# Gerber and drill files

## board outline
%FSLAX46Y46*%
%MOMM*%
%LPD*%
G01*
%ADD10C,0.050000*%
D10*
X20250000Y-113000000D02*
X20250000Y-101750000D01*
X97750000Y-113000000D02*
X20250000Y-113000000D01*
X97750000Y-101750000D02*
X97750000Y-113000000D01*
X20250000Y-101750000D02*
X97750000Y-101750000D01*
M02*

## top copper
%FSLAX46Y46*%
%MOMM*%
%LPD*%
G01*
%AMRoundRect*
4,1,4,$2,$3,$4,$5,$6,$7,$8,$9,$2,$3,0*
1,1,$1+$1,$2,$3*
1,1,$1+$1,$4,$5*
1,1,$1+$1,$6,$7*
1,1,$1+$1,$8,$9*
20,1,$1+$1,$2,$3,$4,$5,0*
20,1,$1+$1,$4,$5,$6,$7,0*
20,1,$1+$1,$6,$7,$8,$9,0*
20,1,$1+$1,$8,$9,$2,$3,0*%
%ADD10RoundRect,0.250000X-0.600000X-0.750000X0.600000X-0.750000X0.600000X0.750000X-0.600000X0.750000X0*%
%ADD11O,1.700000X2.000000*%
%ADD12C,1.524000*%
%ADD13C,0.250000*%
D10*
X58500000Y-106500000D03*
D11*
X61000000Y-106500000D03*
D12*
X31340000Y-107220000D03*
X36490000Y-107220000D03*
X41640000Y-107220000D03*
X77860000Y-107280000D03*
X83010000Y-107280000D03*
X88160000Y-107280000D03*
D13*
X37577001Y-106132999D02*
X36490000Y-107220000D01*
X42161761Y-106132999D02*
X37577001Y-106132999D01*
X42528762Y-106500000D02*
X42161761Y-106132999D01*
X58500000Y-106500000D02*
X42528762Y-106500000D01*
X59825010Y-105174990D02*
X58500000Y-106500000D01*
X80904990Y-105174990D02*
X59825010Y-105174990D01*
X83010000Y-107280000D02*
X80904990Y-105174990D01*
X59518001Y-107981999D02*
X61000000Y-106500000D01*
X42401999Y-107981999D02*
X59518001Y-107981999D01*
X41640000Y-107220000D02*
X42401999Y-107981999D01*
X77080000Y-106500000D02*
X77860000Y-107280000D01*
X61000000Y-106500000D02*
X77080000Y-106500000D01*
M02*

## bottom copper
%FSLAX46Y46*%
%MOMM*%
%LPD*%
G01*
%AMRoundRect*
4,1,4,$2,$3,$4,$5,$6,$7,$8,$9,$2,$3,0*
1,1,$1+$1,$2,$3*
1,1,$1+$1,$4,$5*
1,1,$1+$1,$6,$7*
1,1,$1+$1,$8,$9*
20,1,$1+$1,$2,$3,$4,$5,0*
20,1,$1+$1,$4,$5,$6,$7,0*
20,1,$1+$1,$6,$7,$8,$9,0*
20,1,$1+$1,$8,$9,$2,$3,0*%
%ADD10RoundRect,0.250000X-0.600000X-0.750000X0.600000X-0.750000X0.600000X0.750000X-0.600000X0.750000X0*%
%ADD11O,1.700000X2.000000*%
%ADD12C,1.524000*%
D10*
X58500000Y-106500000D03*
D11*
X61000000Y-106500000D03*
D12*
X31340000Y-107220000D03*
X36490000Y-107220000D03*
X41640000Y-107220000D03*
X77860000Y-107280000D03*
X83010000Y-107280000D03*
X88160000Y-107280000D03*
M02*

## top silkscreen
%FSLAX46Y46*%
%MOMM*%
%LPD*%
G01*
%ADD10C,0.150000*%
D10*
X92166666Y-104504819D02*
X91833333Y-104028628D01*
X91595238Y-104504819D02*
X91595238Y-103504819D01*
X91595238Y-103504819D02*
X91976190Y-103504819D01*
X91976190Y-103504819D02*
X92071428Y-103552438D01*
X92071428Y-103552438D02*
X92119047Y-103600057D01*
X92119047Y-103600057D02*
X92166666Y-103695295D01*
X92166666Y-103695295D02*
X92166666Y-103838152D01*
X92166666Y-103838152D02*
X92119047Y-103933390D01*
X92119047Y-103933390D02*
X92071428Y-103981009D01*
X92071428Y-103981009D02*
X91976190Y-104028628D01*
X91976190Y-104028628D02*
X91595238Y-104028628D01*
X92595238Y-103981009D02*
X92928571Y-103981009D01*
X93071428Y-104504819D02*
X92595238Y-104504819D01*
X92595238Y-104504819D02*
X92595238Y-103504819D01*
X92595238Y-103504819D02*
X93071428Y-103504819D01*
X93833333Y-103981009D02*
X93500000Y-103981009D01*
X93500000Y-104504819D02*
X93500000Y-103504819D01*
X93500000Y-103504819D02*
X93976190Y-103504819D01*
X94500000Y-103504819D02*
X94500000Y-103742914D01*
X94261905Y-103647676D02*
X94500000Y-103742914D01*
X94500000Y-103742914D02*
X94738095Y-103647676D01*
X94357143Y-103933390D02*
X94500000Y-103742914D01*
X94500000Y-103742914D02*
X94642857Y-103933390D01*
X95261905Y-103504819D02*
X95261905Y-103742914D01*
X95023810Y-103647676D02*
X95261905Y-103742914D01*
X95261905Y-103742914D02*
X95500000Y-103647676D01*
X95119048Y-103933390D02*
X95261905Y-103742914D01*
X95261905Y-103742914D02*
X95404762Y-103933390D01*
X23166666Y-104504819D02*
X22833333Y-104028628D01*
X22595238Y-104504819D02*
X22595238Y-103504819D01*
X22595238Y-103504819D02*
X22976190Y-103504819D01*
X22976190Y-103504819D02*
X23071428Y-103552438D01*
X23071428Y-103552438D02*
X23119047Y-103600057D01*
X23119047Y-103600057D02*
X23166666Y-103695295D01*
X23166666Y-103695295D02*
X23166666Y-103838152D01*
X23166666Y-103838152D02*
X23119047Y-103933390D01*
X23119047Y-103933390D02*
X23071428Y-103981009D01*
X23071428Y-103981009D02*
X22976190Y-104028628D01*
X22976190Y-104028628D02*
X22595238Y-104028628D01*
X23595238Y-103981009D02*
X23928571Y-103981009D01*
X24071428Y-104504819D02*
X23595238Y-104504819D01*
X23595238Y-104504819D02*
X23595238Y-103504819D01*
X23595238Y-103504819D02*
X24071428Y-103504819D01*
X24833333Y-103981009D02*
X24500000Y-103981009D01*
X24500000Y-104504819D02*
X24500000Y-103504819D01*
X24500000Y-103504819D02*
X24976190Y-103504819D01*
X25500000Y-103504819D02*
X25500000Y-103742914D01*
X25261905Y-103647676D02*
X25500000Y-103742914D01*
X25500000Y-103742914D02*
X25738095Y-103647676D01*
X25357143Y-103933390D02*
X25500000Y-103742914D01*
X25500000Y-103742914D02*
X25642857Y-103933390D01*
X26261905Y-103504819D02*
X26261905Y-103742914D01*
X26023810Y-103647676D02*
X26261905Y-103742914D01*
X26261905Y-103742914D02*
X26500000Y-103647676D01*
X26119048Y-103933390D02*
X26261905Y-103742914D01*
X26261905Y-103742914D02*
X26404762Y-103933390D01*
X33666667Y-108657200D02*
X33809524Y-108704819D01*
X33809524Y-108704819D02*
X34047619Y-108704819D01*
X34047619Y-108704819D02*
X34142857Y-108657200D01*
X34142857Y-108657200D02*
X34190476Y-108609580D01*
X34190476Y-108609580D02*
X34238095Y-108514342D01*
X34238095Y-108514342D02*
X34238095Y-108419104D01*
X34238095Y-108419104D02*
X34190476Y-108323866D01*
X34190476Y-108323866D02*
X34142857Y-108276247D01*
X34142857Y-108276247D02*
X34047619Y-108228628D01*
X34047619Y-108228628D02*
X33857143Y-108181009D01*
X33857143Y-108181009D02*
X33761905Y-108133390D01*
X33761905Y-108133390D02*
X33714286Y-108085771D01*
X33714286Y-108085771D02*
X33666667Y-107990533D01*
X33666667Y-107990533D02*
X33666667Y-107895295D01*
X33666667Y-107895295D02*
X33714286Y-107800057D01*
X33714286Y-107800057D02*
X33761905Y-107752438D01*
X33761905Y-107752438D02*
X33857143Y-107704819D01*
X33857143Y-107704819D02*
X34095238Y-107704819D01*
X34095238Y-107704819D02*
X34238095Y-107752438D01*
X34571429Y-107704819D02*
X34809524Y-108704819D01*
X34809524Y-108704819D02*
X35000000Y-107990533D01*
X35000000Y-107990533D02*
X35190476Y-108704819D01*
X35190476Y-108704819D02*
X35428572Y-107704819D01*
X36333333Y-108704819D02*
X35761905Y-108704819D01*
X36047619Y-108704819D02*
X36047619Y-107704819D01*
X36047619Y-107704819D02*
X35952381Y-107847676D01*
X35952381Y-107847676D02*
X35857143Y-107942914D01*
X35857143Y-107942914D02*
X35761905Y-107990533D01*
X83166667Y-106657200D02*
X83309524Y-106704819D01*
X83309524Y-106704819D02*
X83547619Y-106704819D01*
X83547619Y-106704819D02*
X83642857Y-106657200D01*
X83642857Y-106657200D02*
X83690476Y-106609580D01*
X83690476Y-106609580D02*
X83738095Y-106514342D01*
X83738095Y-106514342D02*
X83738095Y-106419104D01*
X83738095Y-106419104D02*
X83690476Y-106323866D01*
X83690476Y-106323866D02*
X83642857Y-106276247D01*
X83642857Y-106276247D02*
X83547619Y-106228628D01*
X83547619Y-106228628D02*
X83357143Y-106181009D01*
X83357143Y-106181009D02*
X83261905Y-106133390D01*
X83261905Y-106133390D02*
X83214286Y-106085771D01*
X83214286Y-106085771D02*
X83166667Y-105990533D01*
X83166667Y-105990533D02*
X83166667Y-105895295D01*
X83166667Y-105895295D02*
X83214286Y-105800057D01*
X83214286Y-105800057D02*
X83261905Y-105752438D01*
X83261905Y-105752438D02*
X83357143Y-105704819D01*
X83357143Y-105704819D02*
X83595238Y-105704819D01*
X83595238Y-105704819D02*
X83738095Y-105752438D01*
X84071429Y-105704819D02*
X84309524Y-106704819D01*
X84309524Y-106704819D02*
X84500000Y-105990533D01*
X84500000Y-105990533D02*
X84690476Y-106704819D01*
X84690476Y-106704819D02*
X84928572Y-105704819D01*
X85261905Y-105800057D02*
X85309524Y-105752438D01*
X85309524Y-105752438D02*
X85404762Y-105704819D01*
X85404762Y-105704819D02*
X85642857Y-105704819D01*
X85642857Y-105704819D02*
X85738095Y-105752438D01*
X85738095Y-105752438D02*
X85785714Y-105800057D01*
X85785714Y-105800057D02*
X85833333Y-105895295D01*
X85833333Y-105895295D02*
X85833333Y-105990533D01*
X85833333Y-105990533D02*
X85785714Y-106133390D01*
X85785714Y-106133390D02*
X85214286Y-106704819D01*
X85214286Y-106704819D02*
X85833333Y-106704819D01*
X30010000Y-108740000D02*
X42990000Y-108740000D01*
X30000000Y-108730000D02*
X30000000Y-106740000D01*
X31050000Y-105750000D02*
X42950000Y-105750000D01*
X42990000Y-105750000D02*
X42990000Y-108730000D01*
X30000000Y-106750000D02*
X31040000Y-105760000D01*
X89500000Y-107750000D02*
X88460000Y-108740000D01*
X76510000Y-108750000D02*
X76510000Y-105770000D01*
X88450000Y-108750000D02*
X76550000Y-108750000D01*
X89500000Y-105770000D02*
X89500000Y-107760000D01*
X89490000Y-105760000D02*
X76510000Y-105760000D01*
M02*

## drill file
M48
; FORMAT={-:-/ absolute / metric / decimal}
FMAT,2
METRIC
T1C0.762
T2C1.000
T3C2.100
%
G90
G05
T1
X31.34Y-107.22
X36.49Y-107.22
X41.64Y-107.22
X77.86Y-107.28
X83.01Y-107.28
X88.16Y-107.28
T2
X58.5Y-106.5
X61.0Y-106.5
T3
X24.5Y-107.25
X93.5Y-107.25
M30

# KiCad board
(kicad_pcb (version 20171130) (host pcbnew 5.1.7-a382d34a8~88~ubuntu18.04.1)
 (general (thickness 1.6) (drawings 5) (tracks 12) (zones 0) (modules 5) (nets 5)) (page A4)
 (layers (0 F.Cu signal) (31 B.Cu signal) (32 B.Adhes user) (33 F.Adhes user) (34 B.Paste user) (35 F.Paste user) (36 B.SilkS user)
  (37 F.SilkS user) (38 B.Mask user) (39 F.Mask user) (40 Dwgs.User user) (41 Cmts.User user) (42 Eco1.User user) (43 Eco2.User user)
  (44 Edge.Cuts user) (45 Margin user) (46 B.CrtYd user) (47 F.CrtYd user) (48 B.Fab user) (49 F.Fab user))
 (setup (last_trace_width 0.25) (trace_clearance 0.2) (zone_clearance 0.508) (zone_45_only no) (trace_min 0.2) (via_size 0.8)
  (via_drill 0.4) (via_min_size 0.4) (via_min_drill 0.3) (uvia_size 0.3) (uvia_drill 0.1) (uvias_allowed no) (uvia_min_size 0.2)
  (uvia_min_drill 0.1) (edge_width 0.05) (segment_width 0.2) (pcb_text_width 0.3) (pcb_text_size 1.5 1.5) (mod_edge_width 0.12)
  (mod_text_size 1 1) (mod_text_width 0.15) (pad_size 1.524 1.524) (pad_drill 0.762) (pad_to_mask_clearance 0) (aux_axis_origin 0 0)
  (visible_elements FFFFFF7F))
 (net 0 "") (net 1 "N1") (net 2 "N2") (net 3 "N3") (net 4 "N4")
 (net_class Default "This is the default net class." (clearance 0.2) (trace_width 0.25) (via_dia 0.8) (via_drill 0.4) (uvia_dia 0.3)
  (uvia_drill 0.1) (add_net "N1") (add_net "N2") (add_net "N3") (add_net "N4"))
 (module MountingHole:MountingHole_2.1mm (layer F.Cu) (at 93.5 107.25)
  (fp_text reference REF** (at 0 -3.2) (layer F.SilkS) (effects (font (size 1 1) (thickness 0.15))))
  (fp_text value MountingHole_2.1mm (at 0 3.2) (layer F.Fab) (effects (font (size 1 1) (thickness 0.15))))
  (pad "" np_thru_hole circle (at 0 0) (size 2.1 2.1) (drill 2.1) (layers *.Cu *.Mask)))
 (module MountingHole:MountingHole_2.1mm (layer F.Cu) (at 24.5 107.25)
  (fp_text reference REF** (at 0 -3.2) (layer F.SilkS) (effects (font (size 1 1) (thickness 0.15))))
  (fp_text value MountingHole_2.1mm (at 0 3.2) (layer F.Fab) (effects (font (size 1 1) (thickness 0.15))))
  (pad "" np_thru_hole circle (at 0 0) (size 2.1 2.1) (drill 2.1) (layers *.Cu *.Mask)))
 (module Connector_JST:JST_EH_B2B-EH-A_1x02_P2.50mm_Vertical (layer B.Cu) (at 58.5 106.5)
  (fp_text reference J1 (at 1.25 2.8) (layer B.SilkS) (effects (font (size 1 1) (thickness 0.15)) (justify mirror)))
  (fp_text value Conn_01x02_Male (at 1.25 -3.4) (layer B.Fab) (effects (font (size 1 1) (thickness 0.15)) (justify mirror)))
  (pad 1 thru_hole roundrect (at 0 0) (size 1.7 2) (drill 1) (layers *.Cu *.Mask) (roundrect_rratio 0.147059) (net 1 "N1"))
  (pad 2 thru_hole oval (at 2.5 0) (size 1.7 2) (drill 1) (layers *.Cu *.Mask) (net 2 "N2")))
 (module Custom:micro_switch (layer F.Cu) (at 35 107.75)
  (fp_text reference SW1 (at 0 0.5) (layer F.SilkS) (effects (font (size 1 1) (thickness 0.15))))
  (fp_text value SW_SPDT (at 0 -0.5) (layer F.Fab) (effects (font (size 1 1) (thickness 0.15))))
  (fp_line (start -4.99 0.99) (end 7.99 0.99) (layer F.SilkS) (width 0.15))
  (fp_line (start -5 0.98) (end -5 -1.01) (layer F.SilkS) (width 0.15))
  (fp_line (start -3.95 -2) (end 7.95 -2) (layer F.SilkS) (width 0.15))
  (fp_line (start 7.99 -2) (end 7.99 0.98) (layer F.SilkS) (width 0.15))
  (fp_line (start -5 -1) (end -3.96 -1.99) (layer F.SilkS) (width 0.15))
  (pad 1 thru_hole circle (at -3.66 -0.53) (size 1.524 1.524) (drill 0.762) (layers *.Cu *.Mask) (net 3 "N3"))
  (pad 2 thru_hole circle (at 1.49 -0.53) (size 1.524 1.524) (drill 0.762) (layers *.Cu *.Mask) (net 1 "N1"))
  (pad 3 thru_hole circle (at 6.64 -0.53) (size 1.524 1.524) (drill 0.762) (layers *.Cu *.Mask) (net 2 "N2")))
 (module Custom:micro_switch (layer F.Cu) (at 84.5 106.75 180)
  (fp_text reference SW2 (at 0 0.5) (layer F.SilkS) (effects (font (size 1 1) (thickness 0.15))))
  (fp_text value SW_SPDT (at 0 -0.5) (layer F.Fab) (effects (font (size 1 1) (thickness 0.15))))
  (fp_line (start -5 -1) (end -3.96 -1.99) (layer F.SilkS) (width 0.15))
  (fp_line (start 7.99 -2) (end 7.99 0.98) (layer F.SilkS) (width 0.15))
  (fp_line (start -3.95 -2) (end 7.95 -2) (layer F.SilkS) (width 0.15))
  (fp_line (start -5 0.98) (end -5 -1.01) (layer F.SilkS) (width 0.15))
  (fp_line (start -4.99 0.99) (end 7.99 0.99) (layer F.SilkS) (width 0.15))
  (pad 3 thru_hole circle (at 6.64 -0.53 180) (size 1.524 1.524) (drill 0.762) (layers *.Cu *.Mask) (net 2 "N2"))
  (pad 2 thru_hole circle (at 1.49 -0.53 180) (size 1.524 1.524) (drill 0.762) (layers *.Cu *.Mask) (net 1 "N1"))
  (pad 1 thru_hole circle (at -3.66 -0.53 180) (size 1.524 1.524) (drill 0.762) (layers *.Cu *.Mask) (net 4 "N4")))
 (gr_line (start 20.25 113) (end 20.25 101.75) (layer Edge.Cuts) (width 0.05))
 (gr_line (start 97.75 113) (end 20.25 113) (layer Edge.Cuts) (width 0.05))
 (gr_line (start 97.75 101.75) (end 97.75 113) (layer Edge.Cuts) (width 0.05))
 (gr_line (start 20.25 101.75) (end 97.75 101.75) (layer Edge.Cuts) (width 0.05))
 (segment (start 37.577001 106.132999) (end 36.49 107.22) (width 0.25) (layer F.Cu) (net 1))
 (segment (start 42.161761 106.132999) (end 37.577001 106.132999) (width 0.25) (layer F.Cu) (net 1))
 (segment (start 42.528762 106.5) (end 42.161761 106.132999) (width 0.25) (layer F.Cu) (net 1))
 (segment (start 58.5 106.5) (end 42.528762 106.5) (width 0.25) (layer F.Cu) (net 1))
 (segment (start 59.82501 105.17499) (end 58.5 106.5) (width 0.25) (layer F.Cu) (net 1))
 (segment (start 80.90499 105.17499) (end 59.82501 105.17499) (width 0.25) (layer F.Cu) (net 1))
 (segment (start 83.01 107.28) (end 80.90499 105.17499) (width 0.25) (layer F.Cu) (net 1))
 (segment (start 59.518001 107.981999) (end 61 106.5) (width 0.25) (layer F.Cu) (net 2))
 (segment (start 42.401999 107.981999) (end 59.518001 107.981999) (width 0.25) (layer F.Cu) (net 2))
 (segment (start 41.64 107.22) (end 42.401999 107.981999) (width 0.25) (layer F.Cu) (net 2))
 (segment (start 77.08 106.5) (end 77.86 107.28) (width 0.25) (layer F.Cu) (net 2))
 (segment (start 61 106.5) (end 77.08 106.5) (width 0.25) (layer F.Cu) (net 2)))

